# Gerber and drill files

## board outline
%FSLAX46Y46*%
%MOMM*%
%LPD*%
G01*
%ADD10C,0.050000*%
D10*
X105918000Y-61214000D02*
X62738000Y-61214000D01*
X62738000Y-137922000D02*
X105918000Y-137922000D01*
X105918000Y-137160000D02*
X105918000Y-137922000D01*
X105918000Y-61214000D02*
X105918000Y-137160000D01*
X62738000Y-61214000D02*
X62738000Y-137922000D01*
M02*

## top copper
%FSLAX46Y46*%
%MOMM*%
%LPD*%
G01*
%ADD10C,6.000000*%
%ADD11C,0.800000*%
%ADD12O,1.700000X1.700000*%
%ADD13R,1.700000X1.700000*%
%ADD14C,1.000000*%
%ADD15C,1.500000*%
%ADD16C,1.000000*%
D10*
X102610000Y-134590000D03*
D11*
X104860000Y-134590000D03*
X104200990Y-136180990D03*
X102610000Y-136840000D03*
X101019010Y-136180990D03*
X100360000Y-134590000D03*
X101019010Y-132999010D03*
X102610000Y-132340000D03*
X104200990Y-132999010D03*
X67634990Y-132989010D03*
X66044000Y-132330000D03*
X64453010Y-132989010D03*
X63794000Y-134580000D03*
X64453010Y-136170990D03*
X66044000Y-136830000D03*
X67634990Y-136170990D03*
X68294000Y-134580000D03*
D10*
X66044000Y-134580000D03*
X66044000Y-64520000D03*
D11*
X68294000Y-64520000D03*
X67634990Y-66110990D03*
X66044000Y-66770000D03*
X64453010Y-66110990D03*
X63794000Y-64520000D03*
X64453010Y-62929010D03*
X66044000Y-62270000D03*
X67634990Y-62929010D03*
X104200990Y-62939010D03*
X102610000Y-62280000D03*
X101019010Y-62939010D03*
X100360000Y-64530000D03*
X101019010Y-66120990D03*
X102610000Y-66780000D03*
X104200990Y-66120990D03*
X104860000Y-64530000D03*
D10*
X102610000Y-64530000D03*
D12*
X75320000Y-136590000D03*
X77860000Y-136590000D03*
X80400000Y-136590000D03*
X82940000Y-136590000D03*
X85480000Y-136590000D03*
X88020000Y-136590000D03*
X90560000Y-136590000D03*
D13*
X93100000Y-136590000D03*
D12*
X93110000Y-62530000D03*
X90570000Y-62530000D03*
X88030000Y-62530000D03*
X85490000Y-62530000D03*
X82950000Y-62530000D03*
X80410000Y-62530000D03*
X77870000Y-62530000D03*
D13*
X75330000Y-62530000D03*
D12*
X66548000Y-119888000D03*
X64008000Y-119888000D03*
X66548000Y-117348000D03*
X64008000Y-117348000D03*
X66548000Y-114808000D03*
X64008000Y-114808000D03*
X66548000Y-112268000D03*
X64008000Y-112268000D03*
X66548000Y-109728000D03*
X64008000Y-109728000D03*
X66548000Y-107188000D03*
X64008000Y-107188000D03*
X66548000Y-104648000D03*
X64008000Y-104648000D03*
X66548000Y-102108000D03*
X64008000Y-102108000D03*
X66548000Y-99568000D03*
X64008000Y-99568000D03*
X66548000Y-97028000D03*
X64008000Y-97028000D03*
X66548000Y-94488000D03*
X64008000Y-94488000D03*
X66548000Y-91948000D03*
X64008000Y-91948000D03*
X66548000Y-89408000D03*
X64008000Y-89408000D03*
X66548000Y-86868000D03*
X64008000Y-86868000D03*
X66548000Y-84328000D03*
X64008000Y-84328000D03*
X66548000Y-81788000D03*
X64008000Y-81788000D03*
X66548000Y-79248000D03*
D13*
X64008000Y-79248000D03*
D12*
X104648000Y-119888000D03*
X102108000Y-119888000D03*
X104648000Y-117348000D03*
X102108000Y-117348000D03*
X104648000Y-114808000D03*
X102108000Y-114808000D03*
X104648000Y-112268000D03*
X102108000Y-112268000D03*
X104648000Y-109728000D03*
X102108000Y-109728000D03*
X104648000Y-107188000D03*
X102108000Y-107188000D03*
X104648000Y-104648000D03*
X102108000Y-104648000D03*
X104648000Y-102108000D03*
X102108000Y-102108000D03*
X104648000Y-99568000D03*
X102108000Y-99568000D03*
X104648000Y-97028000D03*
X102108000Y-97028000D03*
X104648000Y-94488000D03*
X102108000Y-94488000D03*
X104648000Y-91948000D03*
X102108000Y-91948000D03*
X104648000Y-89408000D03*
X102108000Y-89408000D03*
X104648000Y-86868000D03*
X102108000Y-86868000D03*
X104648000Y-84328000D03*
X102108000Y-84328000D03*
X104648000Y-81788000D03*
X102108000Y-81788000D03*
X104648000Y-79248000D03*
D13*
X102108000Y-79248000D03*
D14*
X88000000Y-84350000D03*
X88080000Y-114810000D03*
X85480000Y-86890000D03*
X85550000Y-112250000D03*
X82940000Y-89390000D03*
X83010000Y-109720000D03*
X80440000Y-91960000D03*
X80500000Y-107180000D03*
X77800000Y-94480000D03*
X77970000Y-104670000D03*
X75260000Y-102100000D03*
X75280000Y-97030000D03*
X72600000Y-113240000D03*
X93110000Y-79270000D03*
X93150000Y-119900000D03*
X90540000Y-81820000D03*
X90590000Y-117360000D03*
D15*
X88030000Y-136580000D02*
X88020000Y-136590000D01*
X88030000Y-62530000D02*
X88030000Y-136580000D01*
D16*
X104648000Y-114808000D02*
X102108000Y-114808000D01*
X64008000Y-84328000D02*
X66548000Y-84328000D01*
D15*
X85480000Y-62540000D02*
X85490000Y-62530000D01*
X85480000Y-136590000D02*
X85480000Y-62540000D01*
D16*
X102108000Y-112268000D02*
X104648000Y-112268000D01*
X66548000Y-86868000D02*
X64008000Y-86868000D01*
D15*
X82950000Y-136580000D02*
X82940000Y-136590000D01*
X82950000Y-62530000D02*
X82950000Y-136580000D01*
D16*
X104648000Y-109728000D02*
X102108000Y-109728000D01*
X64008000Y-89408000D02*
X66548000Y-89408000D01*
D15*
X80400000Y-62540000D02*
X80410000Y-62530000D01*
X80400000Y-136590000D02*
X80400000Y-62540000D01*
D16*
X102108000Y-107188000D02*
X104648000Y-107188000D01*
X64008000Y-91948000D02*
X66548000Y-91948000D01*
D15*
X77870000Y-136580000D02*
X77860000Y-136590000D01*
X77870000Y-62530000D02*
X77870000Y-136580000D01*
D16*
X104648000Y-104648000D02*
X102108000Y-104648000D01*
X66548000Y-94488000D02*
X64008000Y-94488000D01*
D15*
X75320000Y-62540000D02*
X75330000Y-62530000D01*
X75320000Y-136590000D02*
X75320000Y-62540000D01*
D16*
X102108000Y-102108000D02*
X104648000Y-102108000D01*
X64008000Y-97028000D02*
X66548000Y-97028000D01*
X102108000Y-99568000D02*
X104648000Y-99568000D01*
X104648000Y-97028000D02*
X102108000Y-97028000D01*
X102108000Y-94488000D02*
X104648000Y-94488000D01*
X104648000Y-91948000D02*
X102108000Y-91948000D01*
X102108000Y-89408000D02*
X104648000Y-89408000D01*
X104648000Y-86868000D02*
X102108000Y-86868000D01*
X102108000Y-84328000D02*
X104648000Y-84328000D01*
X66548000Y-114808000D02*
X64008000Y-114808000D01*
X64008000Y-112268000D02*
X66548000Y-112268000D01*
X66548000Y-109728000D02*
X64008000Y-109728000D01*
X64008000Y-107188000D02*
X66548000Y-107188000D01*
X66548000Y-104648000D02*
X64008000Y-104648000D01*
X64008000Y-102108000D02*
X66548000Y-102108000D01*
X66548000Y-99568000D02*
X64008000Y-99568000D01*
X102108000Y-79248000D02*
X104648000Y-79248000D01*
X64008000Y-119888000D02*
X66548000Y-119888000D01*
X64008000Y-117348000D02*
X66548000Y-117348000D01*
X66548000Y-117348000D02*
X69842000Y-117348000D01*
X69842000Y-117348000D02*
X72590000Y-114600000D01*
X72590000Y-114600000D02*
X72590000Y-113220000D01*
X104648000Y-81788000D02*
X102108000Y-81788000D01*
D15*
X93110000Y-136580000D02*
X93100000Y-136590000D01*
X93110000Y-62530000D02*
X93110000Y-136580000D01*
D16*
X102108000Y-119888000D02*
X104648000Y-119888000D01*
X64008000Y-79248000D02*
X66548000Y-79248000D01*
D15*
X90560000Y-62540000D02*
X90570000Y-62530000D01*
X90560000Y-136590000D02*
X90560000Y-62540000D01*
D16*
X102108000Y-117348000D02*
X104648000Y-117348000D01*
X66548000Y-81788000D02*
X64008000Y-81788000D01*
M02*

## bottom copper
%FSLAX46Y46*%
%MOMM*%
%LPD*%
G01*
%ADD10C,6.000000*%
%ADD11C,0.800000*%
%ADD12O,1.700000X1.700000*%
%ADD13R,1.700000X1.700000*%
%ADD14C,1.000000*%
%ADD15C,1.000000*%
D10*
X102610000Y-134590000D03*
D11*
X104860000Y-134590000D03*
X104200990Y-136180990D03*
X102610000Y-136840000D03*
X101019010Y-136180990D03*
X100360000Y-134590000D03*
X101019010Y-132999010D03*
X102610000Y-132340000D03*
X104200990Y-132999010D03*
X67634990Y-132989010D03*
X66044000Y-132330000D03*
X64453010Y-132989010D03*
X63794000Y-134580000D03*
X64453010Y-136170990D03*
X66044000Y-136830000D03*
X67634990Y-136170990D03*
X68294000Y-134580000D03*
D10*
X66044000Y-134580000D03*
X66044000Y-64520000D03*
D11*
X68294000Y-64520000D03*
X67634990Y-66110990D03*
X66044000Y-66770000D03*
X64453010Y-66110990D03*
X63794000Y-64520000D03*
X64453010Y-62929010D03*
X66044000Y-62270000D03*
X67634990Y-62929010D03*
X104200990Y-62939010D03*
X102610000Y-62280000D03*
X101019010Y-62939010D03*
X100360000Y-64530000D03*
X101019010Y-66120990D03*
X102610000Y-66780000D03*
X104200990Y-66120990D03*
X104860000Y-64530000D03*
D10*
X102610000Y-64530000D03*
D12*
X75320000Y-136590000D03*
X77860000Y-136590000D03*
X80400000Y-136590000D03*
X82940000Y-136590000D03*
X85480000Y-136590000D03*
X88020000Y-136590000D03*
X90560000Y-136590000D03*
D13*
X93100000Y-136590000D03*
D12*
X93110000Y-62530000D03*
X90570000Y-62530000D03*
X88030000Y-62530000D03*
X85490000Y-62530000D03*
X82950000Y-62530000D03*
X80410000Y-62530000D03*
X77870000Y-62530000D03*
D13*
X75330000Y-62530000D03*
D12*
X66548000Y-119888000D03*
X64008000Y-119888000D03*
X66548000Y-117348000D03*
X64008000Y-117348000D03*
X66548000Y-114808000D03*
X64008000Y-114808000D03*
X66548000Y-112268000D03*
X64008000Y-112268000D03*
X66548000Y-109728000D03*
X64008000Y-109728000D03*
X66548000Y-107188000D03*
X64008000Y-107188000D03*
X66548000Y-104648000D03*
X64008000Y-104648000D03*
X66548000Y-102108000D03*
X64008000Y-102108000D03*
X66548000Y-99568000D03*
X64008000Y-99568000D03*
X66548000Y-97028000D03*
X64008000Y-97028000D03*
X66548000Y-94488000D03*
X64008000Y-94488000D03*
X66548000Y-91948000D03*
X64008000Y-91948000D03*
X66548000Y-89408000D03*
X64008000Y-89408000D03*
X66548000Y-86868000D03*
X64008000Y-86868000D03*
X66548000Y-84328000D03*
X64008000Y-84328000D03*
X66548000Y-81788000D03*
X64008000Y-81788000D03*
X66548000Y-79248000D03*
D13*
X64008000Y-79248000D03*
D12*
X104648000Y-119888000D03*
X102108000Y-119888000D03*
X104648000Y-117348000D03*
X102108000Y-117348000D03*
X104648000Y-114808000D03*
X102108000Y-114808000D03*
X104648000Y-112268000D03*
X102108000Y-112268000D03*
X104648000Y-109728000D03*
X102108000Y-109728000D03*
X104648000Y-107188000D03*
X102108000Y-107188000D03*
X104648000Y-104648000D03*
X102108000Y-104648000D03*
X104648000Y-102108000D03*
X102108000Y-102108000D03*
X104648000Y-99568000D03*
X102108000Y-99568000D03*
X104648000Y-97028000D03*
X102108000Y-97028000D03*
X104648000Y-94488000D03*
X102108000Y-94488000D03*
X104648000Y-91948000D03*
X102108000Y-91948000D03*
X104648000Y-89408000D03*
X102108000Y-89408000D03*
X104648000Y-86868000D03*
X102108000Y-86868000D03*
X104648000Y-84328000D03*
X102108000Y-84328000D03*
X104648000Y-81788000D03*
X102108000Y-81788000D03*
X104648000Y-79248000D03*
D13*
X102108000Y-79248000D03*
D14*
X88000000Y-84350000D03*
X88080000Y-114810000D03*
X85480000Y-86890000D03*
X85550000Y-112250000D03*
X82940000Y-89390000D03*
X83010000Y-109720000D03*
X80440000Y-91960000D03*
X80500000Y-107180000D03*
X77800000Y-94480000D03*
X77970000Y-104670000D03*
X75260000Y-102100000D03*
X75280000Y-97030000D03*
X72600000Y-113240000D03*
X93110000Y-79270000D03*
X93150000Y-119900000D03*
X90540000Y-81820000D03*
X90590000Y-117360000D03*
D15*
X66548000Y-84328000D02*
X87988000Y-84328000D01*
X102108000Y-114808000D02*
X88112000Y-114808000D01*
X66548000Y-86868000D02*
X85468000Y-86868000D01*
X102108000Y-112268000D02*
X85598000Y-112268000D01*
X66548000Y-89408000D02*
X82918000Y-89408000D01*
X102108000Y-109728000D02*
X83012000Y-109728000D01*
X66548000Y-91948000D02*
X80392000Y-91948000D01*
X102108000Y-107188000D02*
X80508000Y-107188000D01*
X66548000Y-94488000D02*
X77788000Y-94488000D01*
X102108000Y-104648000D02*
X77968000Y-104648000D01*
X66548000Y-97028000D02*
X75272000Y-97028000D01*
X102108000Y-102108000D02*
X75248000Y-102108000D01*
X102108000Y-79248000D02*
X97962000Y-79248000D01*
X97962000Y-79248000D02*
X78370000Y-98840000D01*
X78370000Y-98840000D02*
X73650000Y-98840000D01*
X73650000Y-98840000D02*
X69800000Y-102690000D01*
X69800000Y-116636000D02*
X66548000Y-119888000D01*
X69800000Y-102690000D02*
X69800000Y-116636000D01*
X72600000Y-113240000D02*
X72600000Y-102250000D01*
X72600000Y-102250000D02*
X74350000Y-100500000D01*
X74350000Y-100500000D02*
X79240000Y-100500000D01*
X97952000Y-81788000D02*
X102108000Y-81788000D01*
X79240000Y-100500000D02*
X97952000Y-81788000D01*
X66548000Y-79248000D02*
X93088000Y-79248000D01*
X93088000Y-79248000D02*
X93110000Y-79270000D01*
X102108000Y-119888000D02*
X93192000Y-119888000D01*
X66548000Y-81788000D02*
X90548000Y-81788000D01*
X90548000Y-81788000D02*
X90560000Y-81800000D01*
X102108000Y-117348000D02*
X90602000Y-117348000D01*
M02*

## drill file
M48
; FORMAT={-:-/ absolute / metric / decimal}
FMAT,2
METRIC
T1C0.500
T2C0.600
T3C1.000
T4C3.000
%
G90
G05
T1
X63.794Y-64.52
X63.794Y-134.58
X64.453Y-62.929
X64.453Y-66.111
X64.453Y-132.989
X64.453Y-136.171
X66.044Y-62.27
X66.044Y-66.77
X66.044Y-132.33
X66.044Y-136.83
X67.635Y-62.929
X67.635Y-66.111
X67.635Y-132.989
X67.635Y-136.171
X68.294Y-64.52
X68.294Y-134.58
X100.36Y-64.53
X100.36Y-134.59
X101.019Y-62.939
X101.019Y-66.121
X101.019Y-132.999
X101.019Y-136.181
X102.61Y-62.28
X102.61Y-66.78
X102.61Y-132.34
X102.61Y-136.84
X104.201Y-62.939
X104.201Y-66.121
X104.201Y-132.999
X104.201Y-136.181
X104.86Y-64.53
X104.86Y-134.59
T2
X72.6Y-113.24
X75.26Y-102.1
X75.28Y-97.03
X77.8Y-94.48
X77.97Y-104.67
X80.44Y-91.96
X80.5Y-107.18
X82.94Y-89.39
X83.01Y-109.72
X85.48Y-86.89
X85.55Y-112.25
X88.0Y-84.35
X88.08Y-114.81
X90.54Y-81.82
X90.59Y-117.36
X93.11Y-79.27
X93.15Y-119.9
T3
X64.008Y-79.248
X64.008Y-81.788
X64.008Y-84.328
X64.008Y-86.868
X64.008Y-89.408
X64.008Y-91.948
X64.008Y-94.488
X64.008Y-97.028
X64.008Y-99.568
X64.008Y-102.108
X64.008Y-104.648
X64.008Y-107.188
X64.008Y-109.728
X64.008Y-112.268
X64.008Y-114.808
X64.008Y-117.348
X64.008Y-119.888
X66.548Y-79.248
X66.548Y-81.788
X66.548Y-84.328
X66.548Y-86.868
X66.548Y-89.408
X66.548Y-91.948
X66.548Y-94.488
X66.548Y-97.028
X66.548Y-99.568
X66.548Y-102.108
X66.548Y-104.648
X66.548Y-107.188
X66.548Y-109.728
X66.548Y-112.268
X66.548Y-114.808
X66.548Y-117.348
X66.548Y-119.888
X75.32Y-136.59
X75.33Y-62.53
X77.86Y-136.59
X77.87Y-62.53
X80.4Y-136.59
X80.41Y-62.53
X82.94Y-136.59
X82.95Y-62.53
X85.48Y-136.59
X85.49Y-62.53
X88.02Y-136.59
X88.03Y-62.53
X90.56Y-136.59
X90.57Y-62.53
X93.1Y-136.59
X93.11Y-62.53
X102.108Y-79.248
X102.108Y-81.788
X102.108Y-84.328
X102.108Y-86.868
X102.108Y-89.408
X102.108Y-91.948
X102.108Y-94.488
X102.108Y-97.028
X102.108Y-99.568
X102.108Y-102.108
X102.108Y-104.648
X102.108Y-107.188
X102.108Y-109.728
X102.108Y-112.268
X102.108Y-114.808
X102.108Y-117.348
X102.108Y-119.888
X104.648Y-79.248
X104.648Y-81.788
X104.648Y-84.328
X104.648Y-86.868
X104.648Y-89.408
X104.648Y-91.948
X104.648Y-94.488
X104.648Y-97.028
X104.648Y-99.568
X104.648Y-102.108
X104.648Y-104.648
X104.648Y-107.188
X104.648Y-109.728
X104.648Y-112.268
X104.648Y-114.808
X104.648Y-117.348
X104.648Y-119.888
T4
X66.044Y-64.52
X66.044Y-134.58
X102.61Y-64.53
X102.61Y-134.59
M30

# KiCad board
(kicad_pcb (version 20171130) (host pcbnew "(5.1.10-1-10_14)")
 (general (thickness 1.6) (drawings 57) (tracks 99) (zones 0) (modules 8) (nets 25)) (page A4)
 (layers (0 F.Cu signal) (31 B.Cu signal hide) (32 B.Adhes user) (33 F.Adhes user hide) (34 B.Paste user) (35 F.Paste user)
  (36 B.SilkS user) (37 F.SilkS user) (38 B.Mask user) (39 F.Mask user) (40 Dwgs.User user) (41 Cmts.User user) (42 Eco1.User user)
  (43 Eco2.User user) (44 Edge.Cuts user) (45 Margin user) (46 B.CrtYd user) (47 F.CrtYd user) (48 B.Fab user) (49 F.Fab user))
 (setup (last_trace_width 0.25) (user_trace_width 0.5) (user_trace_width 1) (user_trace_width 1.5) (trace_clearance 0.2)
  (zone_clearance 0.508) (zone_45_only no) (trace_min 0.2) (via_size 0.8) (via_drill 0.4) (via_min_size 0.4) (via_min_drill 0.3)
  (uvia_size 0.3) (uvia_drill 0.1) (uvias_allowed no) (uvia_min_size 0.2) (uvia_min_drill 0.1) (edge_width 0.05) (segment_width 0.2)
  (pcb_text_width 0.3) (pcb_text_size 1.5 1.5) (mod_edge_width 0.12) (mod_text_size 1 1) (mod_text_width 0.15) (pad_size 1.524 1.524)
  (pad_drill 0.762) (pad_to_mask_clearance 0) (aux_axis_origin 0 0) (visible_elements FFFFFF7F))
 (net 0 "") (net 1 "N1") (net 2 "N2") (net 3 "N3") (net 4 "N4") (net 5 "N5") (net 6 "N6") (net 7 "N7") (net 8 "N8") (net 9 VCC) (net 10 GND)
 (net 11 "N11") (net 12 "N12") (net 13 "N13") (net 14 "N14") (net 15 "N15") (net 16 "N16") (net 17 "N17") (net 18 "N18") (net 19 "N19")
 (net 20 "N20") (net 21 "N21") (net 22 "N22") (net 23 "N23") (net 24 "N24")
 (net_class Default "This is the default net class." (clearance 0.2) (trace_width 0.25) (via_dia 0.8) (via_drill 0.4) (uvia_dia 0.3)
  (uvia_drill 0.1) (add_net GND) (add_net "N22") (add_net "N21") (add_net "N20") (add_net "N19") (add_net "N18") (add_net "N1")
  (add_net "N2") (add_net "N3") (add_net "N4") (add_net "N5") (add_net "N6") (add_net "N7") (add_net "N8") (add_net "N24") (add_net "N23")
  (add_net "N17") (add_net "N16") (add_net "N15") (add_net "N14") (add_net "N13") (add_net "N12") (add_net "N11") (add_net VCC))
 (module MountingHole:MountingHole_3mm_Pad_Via (layer F.Cu) (at 102.61 134.59)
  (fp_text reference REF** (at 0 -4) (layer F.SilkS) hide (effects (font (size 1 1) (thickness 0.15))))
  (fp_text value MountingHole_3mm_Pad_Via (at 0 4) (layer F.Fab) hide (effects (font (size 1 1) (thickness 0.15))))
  (pad 1 thru_hole circle (at 0 0) (size 6 6) (drill 3) (layers *.Cu *.Mask))
  (pad 1 thru_hole circle (at 2.25 0) (size 0.8 0.8) (drill 0.5) (layers *.Cu *.Mask))
  (pad 1 thru_hole circle (at 1.59099 1.59099) (size 0.8 0.8) (drill 0.5) (layers *.Cu *.Mask))
  (pad 1 thru_hole circle (at 0 2.25) (size 0.8 0.8) (drill 0.5) (layers *.Cu *.Mask))
  (pad 1 thru_hole circle (at -1.59099 1.59099) (size 0.8 0.8) (drill 0.5) (layers *.Cu *.Mask))
  (pad 1 thru_hole circle (at -2.25 0) (size 0.8 0.8) (drill 0.5) (layers *.Cu *.Mask))
  (pad 1 thru_hole circle (at -1.59099 -1.59099) (size 0.8 0.8) (drill 0.5) (layers *.Cu *.Mask))
  (pad 1 thru_hole circle (at 0 -2.25) (size 0.8 0.8) (drill 0.5) (layers *.Cu *.Mask))
  (pad 1 thru_hole circle (at 1.59099 -1.59099) (size 0.8 0.8) (drill 0.5) (layers *.Cu *.Mask)))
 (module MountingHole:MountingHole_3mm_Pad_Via (layer F.Cu) (at 66.044 134.58)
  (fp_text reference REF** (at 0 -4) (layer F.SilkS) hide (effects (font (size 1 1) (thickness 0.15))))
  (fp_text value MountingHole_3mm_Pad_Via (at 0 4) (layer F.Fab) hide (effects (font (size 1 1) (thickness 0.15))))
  (pad 1 thru_hole circle (at 1.59099 -1.59099) (size 0.8 0.8) (drill 0.5) (layers *.Cu *.Mask))
  (pad 1 thru_hole circle (at 0 -2.25) (size 0.8 0.8) (drill 0.5) (layers *.Cu *.Mask))
  (pad 1 thru_hole circle (at -1.59099 -1.59099) (size 0.8 0.8) (drill 0.5) (layers *.Cu *.Mask))
  (pad 1 thru_hole circle (at -2.25 0) (size 0.8 0.8) (drill 0.5) (layers *.Cu *.Mask))
  (pad 1 thru_hole circle (at -1.59099 1.59099) (size 0.8 0.8) (drill 0.5) (layers *.Cu *.Mask))
  (pad 1 thru_hole circle (at 0 2.25) (size 0.8 0.8) (drill 0.5) (layers *.Cu *.Mask))
  (pad 1 thru_hole circle (at 1.59099 1.59099) (size 0.8 0.8) (drill 0.5) (layers *.Cu *.Mask))
  (pad 1 thru_hole circle (at 2.25 0) (size 0.8 0.8) (drill 0.5) (layers *.Cu *.Mask))
  (pad 1 thru_hole circle (at 0 0) (size 6 6) (drill 3) (layers *.Cu *.Mask)))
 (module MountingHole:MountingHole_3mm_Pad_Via (layer F.Cu) (at 66.044 64.52)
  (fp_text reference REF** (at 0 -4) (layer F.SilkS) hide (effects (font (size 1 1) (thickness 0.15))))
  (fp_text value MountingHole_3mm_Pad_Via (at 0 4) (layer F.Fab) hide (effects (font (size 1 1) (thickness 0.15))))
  (pad 1 thru_hole circle (at 0 0) (size 6 6) (drill 3) (layers *.Cu *.Mask))
  (pad 1 thru_hole circle (at 2.25 0) (size 0.8 0.8) (drill 0.5) (layers *.Cu *.Mask))
  (pad 1 thru_hole circle (at 1.59099 1.59099) (size 0.8 0.8) (drill 0.5) (layers *.Cu *.Mask))
  (pad 1 thru_hole circle (at 0 2.25) (size 0.8 0.8) (drill 0.5) (layers *.Cu *.Mask))
  (pad 1 thru_hole circle (at -1.59099 1.59099) (size 0.8 0.8) (drill 0.5) (layers *.Cu *.Mask))
  (pad 1 thru_hole circle (at -2.25 0) (size 0.8 0.8) (drill 0.5) (layers *.Cu *.Mask))
  (pad 1 thru_hole circle (at -1.59099 -1.59099) (size 0.8 0.8) (drill 0.5) (layers *.Cu *.Mask))
  (pad 1 thru_hole circle (at 0 -2.25) (size 0.8 0.8) (drill 0.5) (layers *.Cu *.Mask))
  (pad 1 thru_hole circle (at 1.59099 -1.59099) (size 0.8 0.8) (drill 0.5) (layers *.Cu *.Mask)))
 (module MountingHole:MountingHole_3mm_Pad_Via (layer F.Cu) (at 102.61 64.53)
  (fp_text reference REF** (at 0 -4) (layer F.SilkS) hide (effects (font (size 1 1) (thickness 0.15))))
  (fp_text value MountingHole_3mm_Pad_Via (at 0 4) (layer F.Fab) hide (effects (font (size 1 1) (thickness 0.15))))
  (pad 1 thru_hole circle (at 1.59099 -1.59099) (size 0.8 0.8) (drill 0.5) (layers *.Cu *.Mask))
  (pad 1 thru_hole circle (at 0 -2.25) (size 0.8 0.8) (drill 0.5) (layers *.Cu *.Mask))
  (pad 1 thru_hole circle (at -1.59099 -1.59099) (size 0.8 0.8) (drill 0.5) (layers *.Cu *.Mask))
  (pad 1 thru_hole circle (at -2.25 0) (size 0.8 0.8) (drill 0.5) (layers *.Cu *.Mask))
  (pad 1 thru_hole circle (at -1.59099 1.59099) (size 0.8 0.8) (drill 0.5) (layers *.Cu *.Mask))
  (pad 1 thru_hole circle (at 0 2.25) (size 0.8 0.8) (drill 0.5) (layers *.Cu *.Mask))
  (pad 1 thru_hole circle (at 1.59099 1.59099) (size 0.8 0.8) (drill 0.5) (layers *.Cu *.Mask))
  (pad 1 thru_hole circle (at 2.25 0) (size 0.8 0.8) (drill 0.5) (layers *.Cu *.Mask))
  (pad 1 thru_hole circle (at 0 0) (size 6 6) (drill 3) (layers *.Cu *.Mask)))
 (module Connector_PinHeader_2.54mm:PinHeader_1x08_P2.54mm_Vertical (layer F.Cu) (at 93.1 136.59 270)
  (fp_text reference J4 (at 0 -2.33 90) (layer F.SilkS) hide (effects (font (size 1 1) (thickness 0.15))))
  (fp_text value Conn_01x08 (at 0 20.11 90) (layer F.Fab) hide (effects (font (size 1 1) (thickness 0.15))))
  (pad 8 thru_hole oval (at 0 17.78 270) (size 1.7 1.7) (drill 1) (layers *.Cu *.Mask) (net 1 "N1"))
  (pad 7 thru_hole oval (at 0 15.24 270) (size 1.7 1.7) (drill 1) (layers *.Cu *.Mask) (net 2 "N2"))
  (pad 6 thru_hole oval (at 0 12.7 270) (size 1.7 1.7) (drill 1) (layers *.Cu *.Mask) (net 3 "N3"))
  (pad 5 thru_hole oval (at 0 10.16 270) (size 1.7 1.7) (drill 1) (layers *.Cu *.Mask) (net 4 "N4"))
  (pad 4 thru_hole oval (at 0 7.62 270) (size 1.7 1.7) (drill 1) (layers *.Cu *.Mask) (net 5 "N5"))
  (pad 3 thru_hole oval (at 0 5.08 270) (size 1.7 1.7) (drill 1) (layers *.Cu *.Mask) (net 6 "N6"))
  (pad 2 thru_hole oval (at 0 2.54 270) (size 1.7 1.7) (drill 1) (layers *.Cu *.Mask) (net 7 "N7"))
  (pad 1 thru_hole rect (at 0 0 270) (size 1.7 1.7) (drill 1) (layers *.Cu *.Mask) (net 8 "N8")))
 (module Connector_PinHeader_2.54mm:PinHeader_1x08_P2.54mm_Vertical (layer F.Cu) (at 75.33 62.53 90)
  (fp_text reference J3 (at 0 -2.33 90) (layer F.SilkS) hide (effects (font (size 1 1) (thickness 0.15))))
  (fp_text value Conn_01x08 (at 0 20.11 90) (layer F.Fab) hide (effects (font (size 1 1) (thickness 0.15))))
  (pad 8 thru_hole oval (at 0 17.78 90) (size 1.7 1.7) (drill 1) (layers *.Cu *.Mask) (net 8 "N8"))
  (pad 7 thru_hole oval (at 0 15.24 90) (size 1.7 1.7) (drill 1) (layers *.Cu *.Mask) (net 7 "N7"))
  (pad 6 thru_hole oval (at 0 12.7 90) (size 1.7 1.7) (drill 1) (layers *.Cu *.Mask) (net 6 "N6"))
  (pad 5 thru_hole oval (at 0 10.16 90) (size 1.7 1.7) (drill 1) (layers *.Cu *.Mask) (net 5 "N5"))
  (pad 4 thru_hole oval (at 0 7.62 90) (size 1.7 1.7) (drill 1) (layers *.Cu *.Mask) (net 4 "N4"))
  (pad 3 thru_hole oval (at 0 5.08 90) (size 1.7 1.7) (drill 1) (layers *.Cu *.Mask) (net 3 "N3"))
  (pad 2 thru_hole oval (at 0 2.54 90) (size 1.7 1.7) (drill 1) (layers *.Cu *.Mask) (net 2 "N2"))
  (pad 1 thru_hole rect (at 0 0 90) (size 1.7 1.7) (drill 1) (layers *.Cu *.Mask) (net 1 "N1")))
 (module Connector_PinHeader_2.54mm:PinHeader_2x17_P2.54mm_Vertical (layer F.Cu) (at 64.008 79.248)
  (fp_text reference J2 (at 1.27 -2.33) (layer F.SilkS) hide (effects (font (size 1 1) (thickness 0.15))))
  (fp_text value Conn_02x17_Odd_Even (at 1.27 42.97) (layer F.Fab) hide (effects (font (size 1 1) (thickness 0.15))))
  (pad 34 thru_hole oval (at 2.54 40.64) (size 1.7 1.7) (drill 1) (layers *.Cu *.Mask) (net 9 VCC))
  (pad 33 thru_hole oval (at 0 40.64) (size 1.7 1.7) (drill 1) (layers *.Cu *.Mask) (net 9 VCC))
  (pad 32 thru_hole oval (at 2.54 38.1) (size 1.7 1.7) (drill 1) (layers *.Cu *.Mask) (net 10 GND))
  (pad 31 thru_hole oval (at 0 38.1) (size 1.7 1.7) (drill 1) (layers *.Cu *.Mask) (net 10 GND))
  (pad 30 thru_hole oval (at 2.54 35.56) (size 1.7 1.7) (drill 1) (layers *.Cu *.Mask) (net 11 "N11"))
  (pad 29 thru_hole oval (at 0 35.56) (size 1.7 1.7) (drill 1) (layers *.Cu *.Mask) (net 11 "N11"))
  (pad 28 thru_hole oval (at 2.54 33.02) (size 1.7 1.7) (drill 1) (layers *.Cu *.Mask) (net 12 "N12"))
  (pad 27 thru_hole oval (at 0 33.02) (size 1.7 1.7) (drill 1) (layers *.Cu *.Mask) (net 12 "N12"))
  (pad 26 thru_hole oval (at 2.54 30.48) (size 1.7 1.7) (drill 1) (layers *.Cu *.Mask) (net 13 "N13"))
  (pad 25 thru_hole oval (at 0 30.48) (size 1.7 1.7) (drill 1) (layers *.Cu *.Mask) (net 13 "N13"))
  (pad 24 thru_hole oval (at 2.54 27.94) (size 1.7 1.7) (drill 1) (layers *.Cu *.Mask) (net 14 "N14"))
  (pad 23 thru_hole oval (at 0 27.94) (size 1.7 1.7) (drill 1) (layers *.Cu *.Mask) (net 14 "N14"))
  (pad 22 thru_hole oval (at 2.54 25.4) (size 1.7 1.7) (drill 1) (layers *.Cu *.Mask) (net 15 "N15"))
  (pad 21 thru_hole oval (at 0 25.4) (size 1.7 1.7) (drill 1) (layers *.Cu *.Mask) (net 15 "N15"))
  (pad 20 thru_hole oval (at 2.54 22.86) (size 1.7 1.7) (drill 1) (layers *.Cu *.Mask) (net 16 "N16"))
  (pad 19 thru_hole oval (at 0 22.86) (size 1.7 1.7) (drill 1) (layers *.Cu *.Mask) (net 16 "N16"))
  (pad 18 thru_hole oval (at 2.54 20.32) (size 1.7 1.7) (drill 1) (layers *.Cu *.Mask) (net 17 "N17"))
  (pad 17 thru_hole oval (at 0 20.32) (size 1.7 1.7) (drill 1) (layers *.Cu *.Mask) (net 17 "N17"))
  (pad 16 thru_hole oval (at 2.54 17.78) (size 1.7 1.7) (drill 1) (layers *.Cu *.Mask) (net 1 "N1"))
  (pad 15 thru_hole oval (at 0 17.78) (size 1.7 1.7) (drill 1) (layers *.Cu *.Mask) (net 1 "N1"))
  (pad 14 thru_hole oval (at 2.54 15.24) (size 1.7 1.7) (drill 1) (layers *.Cu *.Mask) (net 2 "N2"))
  (pad 13 thru_hole oval (at 0 15.24) (size 1.7 1.7) (drill 1) (layers *.Cu *.Mask) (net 2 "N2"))
  (pad 12 thru_hole oval (at 2.54 12.7) (size 1.7 1.7) (drill 1) (layers *.Cu *.Mask) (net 3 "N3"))
  (pad 11 thru_hole oval (at 0 12.7) (size 1.7 1.7) (drill 1) (layers *.Cu *.Mask) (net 3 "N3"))
  (pad 10 thru_hole oval (at 2.54 10.16) (size 1.7 1.7) (drill 1) (layers *.Cu *.Mask) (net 4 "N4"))
  (pad 9 thru_hole oval (at 0 10.16) (size 1.7 1.7) (drill 1) (layers *.Cu *.Mask) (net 4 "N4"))
  (pad 8 thru_hole oval (at 2.54 7.62) (size 1.7 1.7) (drill 1) (layers *.Cu *.Mask) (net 5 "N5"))
  (pad 7 thru_hole oval (at 0 7.62) (size 1.7 1.7) (drill 1) (layers *.Cu *.Mask) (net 5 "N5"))
  (pad 6 thru_hole oval (at 2.54 5.08) (size 1.7 1.7) (drill 1) (layers *.Cu *.Mask) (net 6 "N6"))
  (pad 5 thru_hole oval (at 0 5.08) (size 1.7 1.7) (drill 1) (layers *.Cu *.Mask) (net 6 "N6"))
  (pad 4 thru_hole oval (at 2.54 2.54) (size 1.7 1.7) (drill 1) (layers *.Cu *.Mask) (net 7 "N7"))
  (pad 3 thru_hole oval (at 0 2.54) (size 1.7 1.7) (drill 1) (layers *.Cu *.Mask) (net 7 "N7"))
  (pad 2 thru_hole oval (at 2.54 0) (size 1.7 1.7) (drill 1) (layers *.Cu *.Mask) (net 8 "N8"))
  (pad 1 thru_hole rect (at 0 0) (size 1.7 1.7) (drill 1) (layers *.Cu *.Mask) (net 8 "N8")))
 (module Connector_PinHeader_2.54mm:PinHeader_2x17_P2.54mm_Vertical (layer F.Cu) (at 102.108 79.248)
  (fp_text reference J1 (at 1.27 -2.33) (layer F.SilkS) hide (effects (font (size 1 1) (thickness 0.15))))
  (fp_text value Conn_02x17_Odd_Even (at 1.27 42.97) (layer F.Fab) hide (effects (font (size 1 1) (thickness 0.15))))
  (pad 34 thru_hole oval (at 2.54 40.64) (size 1.7 1.7) (drill 1) (layers *.Cu *.Mask) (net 8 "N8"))
  (pad 33 thru_hole oval (at 0 40.64) (size 1.7 1.7) (drill 1) (layers *.Cu *.Mask) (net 8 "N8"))
  (pad 32 thru_hole oval (at 2.54 38.1) (size 1.7 1.7) (drill 1) (layers *.Cu *.Mask) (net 7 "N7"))
  (pad 31 thru_hole oval (at 0 38.1) (size 1.7 1.7) (drill 1) (layers *.Cu *.Mask) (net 7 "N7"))
  (pad 30 thru_hole oval (at 2.54 35.56) (size 1.7 1.7) (drill 1) (layers *.Cu *.Mask) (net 6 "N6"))
  (pad 29 thru_hole oval (at 0 35.56) (size 1.7 1.7) (drill 1) (layers *.Cu *.Mask) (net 6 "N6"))
  (pad 28 thru_hole oval (at 2.54 33.02) (size 1.7 1.7) (drill 1) (layers *.Cu *.Mask) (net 5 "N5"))
  (pad 27 thru_hole oval (at 0 33.02) (size 1.7 1.7) (drill 1) (layers *.Cu *.Mask) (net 5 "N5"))
  (pad 26 thru_hole oval (at 2.54 30.48) (size 1.7 1.7) (drill 1) (layers *.Cu *.Mask) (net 4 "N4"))
  (pad 25 thru_hole oval (at 0 30.48) (size 1.7 1.7) (drill 1) (layers *.Cu *.Mask) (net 4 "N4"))
  (pad 24 thru_hole oval (at 2.54 27.94) (size 1.7 1.7) (drill 1) (layers *.Cu *.Mask) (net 3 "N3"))
  (pad 23 thru_hole oval (at 0 27.94) (size 1.7 1.7) (drill 1) (layers *.Cu *.Mask) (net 3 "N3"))
  (pad 22 thru_hole oval (at 2.54 25.4) (size 1.7 1.7) (drill 1) (layers *.Cu *.Mask) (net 2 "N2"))
  (pad 21 thru_hole oval (at 0 25.4) (size 1.7 1.7) (drill 1) (layers *.Cu *.Mask) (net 2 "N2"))
  (pad 20 thru_hole oval (at 2.54 22.86) (size 1.7 1.7) (drill 1) (layers *.Cu *.Mask) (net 1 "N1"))
  (pad 19 thru_hole oval (at 0 22.86) (size 1.7 1.7) (drill 1) (layers *.Cu *.Mask) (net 1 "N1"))
  (pad 18 thru_hole oval (at 2.54 20.32) (size 1.7 1.7) (drill 1) (layers *.Cu *.Mask) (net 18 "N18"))
  (pad 17 thru_hole oval (at 0 20.32) (size 1.7 1.7) (drill 1) (layers *.Cu *.Mask) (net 18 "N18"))
  (pad 16 thru_hole oval (at 2.54 17.78) (size 1.7 1.7) (drill 1) (layers *.Cu *.Mask) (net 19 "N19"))
  (pad 15 thru_hole oval (at 0 17.78) (size 1.7 1.7) (drill 1) (layers *.Cu *.Mask) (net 19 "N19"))
  (pad 14 thru_hole oval (at 2.54 15.24) (size 1.7 1.7) (drill 1) (layers *.Cu *.Mask) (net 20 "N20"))
  (pad 13 thru_hole oval (at 0 15.24) (size 1.7 1.7) (drill 1) (layers *.Cu *.Mask) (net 20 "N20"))
  (pad 12 thru_hole oval (at 2.54 12.7) (size 1.7 1.7) (drill 1) (layers *.Cu *.Mask) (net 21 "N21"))
  (pad 11 thru_hole oval (at 0 12.7) (size 1.7 1.7) (drill 1) (layers *.Cu *.Mask) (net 21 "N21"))
  (pad 10 thru_hole oval (at 2.54 10.16) (size 1.7 1.7) (drill 1) (layers *.Cu *.Mask) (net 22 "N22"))
  (pad 9 thru_hole oval (at 0 10.16) (size 1.7 1.7) (drill 1) (layers *.Cu *.Mask) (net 22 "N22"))
  (pad 8 thru_hole oval (at 2.54 7.62) (size 1.7 1.7) (drill 1) (layers *.Cu *.Mask) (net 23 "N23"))
  (pad 7 thru_hole oval (at 0 7.62) (size 1.7 1.7) (drill 1) (layers *.Cu *.Mask) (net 23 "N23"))
  (pad 6 thru_hole oval (at 2.54 5.08) (size 1.7 1.7) (drill 1) (layers *.Cu *.Mask) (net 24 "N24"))
  (pad 5 thru_hole oval (at 0 5.08) (size 1.7 1.7) (drill 1) (layers *.Cu *.Mask) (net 24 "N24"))
  (pad 4 thru_hole oval (at 2.54 2.54) (size 1.7 1.7) (drill 1) (layers *.Cu *.Mask) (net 10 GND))
  (pad 3 thru_hole oval (at 0 2.54) (size 1.7 1.7) (drill 1) (layers *.Cu *.Mask) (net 10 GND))
  (pad 2 thru_hole oval (at 2.54 0) (size 1.7 1.7) (drill 1) (layers *.Cu *.Mask) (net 9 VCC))
  (pad 1 thru_hole rect (at 0 0) (size 1.7 1.7) (drill 1) (layers *.Cu *.Mask) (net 9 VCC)))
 (gr_line (start 105.918 61.214) (end 62.738 61.214) (layer Edge.Cuts) (width 0.05))
 (gr_line (start 62.738 137.922) (end 105.918 137.922) (layer Edge.Cuts) (width 0.05))
 (gr_line (start 105.918 137.16) (end 105.918 137.922) (layer Edge.Cuts) (width 0.05))
 (gr_line (start 105.918 61.214) (end 105.918 137.16) (layer Edge.Cuts) (width 0.05))
 (gr_line (start 62.738 61.214) (end 62.738 137.922) (layer Edge.Cuts) (width 0.05))
 (segment (start 88.03 136.58) (end 88.02 136.59) (width 1.5) (layer F.Cu) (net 6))
 (segment (start 88.03 62.53) (end 88.03 136.58) (width 1.5) (layer F.Cu) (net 6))
 (segment (start 66.548 84.328) (end 87.988 84.328) (width 1) (layer B.Cu) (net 6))
 (via (at 88 84.35) (size 1) (drill 0.6) (layers F.Cu B.Cu) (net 6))
 (segment (start 102.108 114.808) (end 88.112 114.808) (width 1) (layer B.Cu) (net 6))
 (via (at 88.08 114.81) (size 1) (drill 0.6) (layers F.Cu B.Cu) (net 6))
 (segment (start 104.648 114.808) (end 102.108 114.808) (width 1) (layer F.Cu) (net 6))
 (segment (start 64.008 84.328) (end 66.548 84.328) (width 1) (layer F.Cu) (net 6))
 (segment (start 85.48 62.54) (end 85.49 62.53) (width 1.5) (layer F.Cu) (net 5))
 (segment (start 85.48 136.59) (end 85.48 62.54) (width 1.5) (layer F.Cu) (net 5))
 (via (at 85.48 86.89) (size 1) (drill 0.6) (layers F.Cu B.Cu) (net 5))
 (segment (start 66.548 86.868) (end 85.468 86.868) (width 1) (layer B.Cu) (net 5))
 (segment (start 102.108 112.268) (end 85.598 112.268) (width 1) (layer B.Cu) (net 5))
 (via (at 85.55 112.25) (size 1) (drill 0.6) (layers F.Cu B.Cu) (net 5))
 (segment (start 102.108 112.268) (end 104.648 112.268) (width 1) (layer F.Cu) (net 5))
 (segment (start 66.548 86.868) (end 64.008 86.868) (width 1) (layer F.Cu) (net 5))
 (segment (start 82.95 136.58) (end 82.94 136.59) (width 1.5) (layer F.Cu) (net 4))
 (segment (start 82.95 62.53) (end 82.95 136.58) (width 1.5) (layer F.Cu) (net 4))
 (via (at 82.94 89.39) (size 1) (drill 0.6) (layers F.Cu B.Cu) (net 4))
 (segment (start 66.548 89.408) (end 82.918 89.408) (width 1) (layer B.Cu) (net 4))
 (segment (start 102.108 109.728) (end 83.012 109.728) (width 1) (layer B.Cu) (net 4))
 (via (at 83.01 109.72) (size 1) (drill 0.6) (layers F.Cu B.Cu) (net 4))
 (segment (start 104.648 109.728) (end 102.108 109.728) (width 1) (layer F.Cu) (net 4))
 (segment (start 64.008 89.408) (end 66.548 89.408) (width 1) (layer F.Cu) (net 4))
 (segment (start 80.4 62.54) (end 80.41 62.53) (width 1.5) (layer F.Cu) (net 3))
 (segment (start 80.4 136.59) (end 80.4 62.54) (width 1.5) (layer F.Cu) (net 3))
 (via (at 80.44 91.96) (size 1) (drill 0.6) (layers F.Cu B.Cu) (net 3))
 (segment (start 66.548 91.948) (end 80.392 91.948) (width 1) (layer B.Cu) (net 3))
 (segment (start 102.108 107.188) (end 80.508 107.188) (width 1) (layer B.Cu) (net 3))
 (via (at 80.5 107.18) (size 1) (drill 0.6) (layers F.Cu B.Cu) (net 3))
 (segment (start 102.108 107.188) (end 104.648 107.188) (width 1) (layer F.Cu) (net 3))
 (segment (start 64.008 91.948) (end 66.548 91.948) (width 1) (layer F.Cu) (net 3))
 (segment (start 77.87 136.58) (end 77.86 136.59) (width 1.5) (layer F.Cu) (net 2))
 (segment (start 77.87 62.53) (end 77.87 136.58) (width 1.5) (layer F.Cu) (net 2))
 (via (at 77.8 94.48) (size 1) (drill 0.6) (layers F.Cu B.Cu) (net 2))
 (segment (start 66.548 94.488) (end 77.788 94.488) (width 1) (layer B.Cu) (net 2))
 (segment (start 102.108 104.648) (end 77.968 104.648) (width 1) (layer B.Cu) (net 2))
 (via (at 77.97 104.67) (size 1) (drill 0.6) (layers F.Cu B.Cu) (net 2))
 (segment (start 104.648 104.648) (end 102.108 104.648) (width 1) (layer F.Cu) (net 2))
 (segment (start 66.548 94.488) (end 64.008 94.488) (width 1) (layer F.Cu) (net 2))
 (segment (start 75.32 62.54) (end 75.33 62.53) (width 1.5) (layer F.Cu) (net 1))
 (segment (start 75.32 136.59) (end 75.32 62.54) (width 1.5) (layer F.Cu) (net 1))
 (via (at 75.26 102.1) (size 1) (drill 0.6) (layers F.Cu B.Cu) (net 1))
 (via (at 75.28 97.03) (size 1) (drill 0.6) (layers F.Cu B.Cu) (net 1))
 (segment (start 66.548 97.028) (end 75.272 97.028) (width 1) (layer B.Cu) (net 1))
 (segment (start 102.108 102.108) (end 75.248 102.108) (width 1) (layer B.Cu) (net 1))
 (segment (start 102.108 102.108) (end 104.648 102.108) (width 1) (layer F.Cu) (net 1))
 (segment (start 64.008 97.028) (end 66.548 97.028) (width 1) (layer F.Cu) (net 1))
 (segment (start 102.108 99.568) (end 104.648 99.568) (width 1) (layer F.Cu) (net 18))
 (segment (start 104.648 97.028) (end 102.108 97.028) (width 1) (layer F.Cu) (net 19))
 (segment (start 102.108 94.488) (end 104.648 94.488) (width 1) (layer F.Cu) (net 20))
 (segment (start 104.648 91.948) (end 102.108 91.948) (width 1) (layer F.Cu) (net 21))
 (segment (start 102.108 89.408) (end 104.648 89.408) (width 1) (layer F.Cu) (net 22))
 (segment (start 104.648 86.868) (end 102.108 86.868) (width 1) (layer F.Cu) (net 23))
 (segment (start 102.108 84.328) (end 104.648 84.328) (width 1) (layer F.Cu) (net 24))
 (segment (start 66.548 114.808) (end 64.008 114.808) (width 1) (layer F.Cu) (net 11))
 (segment (start 64.008 112.268) (end 66.548 112.268) (width 1) (layer F.Cu) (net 12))
 (segment (start 66.548 109.728) (end 64.008 109.728) (width 1) (layer F.Cu) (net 13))
 (segment (start 64.008 107.188) (end 66.548 107.188) (width 1) (layer F.Cu) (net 14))
 (segment (start 66.548 104.648) (end 64.008 104.648) (width 1) (layer F.Cu) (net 15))
 (segment (start 64.008 102.108) (end 66.548 102.108) (width 1) (layer F.Cu) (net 16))
 (segment (start 66.548 99.568) (end 64.008 99.568) (width 1) (layer F.Cu) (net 17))
 (segment (start 102.108 79.248) (end 97.962 79.248) (width 1) (layer B.Cu) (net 9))
 (segment (start 97.962 79.248) (end 78.37 98.84) (width 1) (layer B.Cu) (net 9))
 (segment (start 78.37 98.84) (end 73.65 98.84) (width 1) (layer B.Cu) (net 9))
 (segment (start 73.65 98.84) (end 69.8 102.69) (width 1) (layer B.Cu) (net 9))
 (segment (start 69.8 116.636) (end 66.548 119.888) (width 1) (layer B.Cu) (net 9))
 (segment (start 69.8 102.69) (end 69.8 116.636) (width 1) (layer B.Cu) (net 9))
 (segment (start 102.108 79.248) (end 104.648 79.248) (width 1) (layer F.Cu) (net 9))
 (segment (start 64.008 119.888) (end 66.548 119.888) (width 1) (layer F.Cu) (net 9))
 (via (at 72.6 113.24) (size 1) (drill 0.6) (layers F.Cu B.Cu) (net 10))
 (segment (start 64.008 117.348) (end 66.548 117.348) (width 1) (layer F.Cu) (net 10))
 (segment (start 66.548 117.348) (end 69.842 117.348) (width 1) (layer F.Cu) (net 10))
 (segment (start 69.842 117.348) (end 72.59 114.6) (width 1) (layer F.Cu) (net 10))
 (segment (start 72.59 114.6) (end 72.59 113.22) (width 1) (layer F.Cu) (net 10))
 (segment (start 72.6 113.24) (end 72.6 102.25) (width 1) (layer B.Cu) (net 10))
 (segment (start 72.6 102.25) (end 74.35 100.5) (width 1) (layer B.Cu) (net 10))
 (segment (start 74.35 100.5) (end 79.24 100.5) (width 1) (layer B.Cu) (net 10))
 (segment (start 97.952 81.788) (end 102.108 81.788) (width 1) (layer B.Cu) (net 10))
 (segment (start 79.24 100.5) (end 97.952 81.788) (width 1) (layer B.Cu) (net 10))
 (segment (start 104.648 81.788) (end 102.108 81.788) (width 1) (layer F.Cu) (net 10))
 (segment (start 93.11 136.58) (end 93.1 136.59) (width 1.5) (layer F.Cu) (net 8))
 (segment (start 93.11 62.53) (end 93.11 136.58) (width 1.5) (layer F.Cu) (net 8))
 (via (at 93.11 79.27) (size 1) (drill 0.6) (layers F.Cu B.Cu) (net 8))
 (segment (start 66.548 79.248) (end 93.088 79.248) (width 1) (layer B.Cu) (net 8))
 (segment (start 93.088 79.248) (end 93.11 79.27) (width 1) (layer B.Cu) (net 8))
 (segment (start 102.108 119.888) (end 93.192 119.888) (width 1) (layer B.Cu) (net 8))
 (via (at 93.15 119.9) (size 1) (drill 0.6) (layers F.Cu B.Cu) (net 8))
 (segment (start 102.108 119.888) (end 104.648 119.888) (width 1) (layer F.Cu) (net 8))
 (segment (start 64.008 79.248) (end 66.548 79.248) (width 1) (layer F.Cu) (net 8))
 (via (at 90.54 81.82) (size 1) (drill 0.6) (layers F.Cu B.Cu) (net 7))
 (segment (start 90.56 62.54) (end 90.57 62.53) (width 1.5) (layer F.Cu) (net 7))
 (segment (start 90.56 136.59) (end 90.56 62.54) (width 1.5) (layer F.Cu) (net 7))
 (segment (start 66.548 81.788) (end 90.548 81.788) (width 1) (layer B.Cu) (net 7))
 (segment (start 90.548 81.788) (end 90.56 81.8) (width 1) (layer B.Cu) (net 7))
 (via (at 90.59 117.36) (size 1) (drill 0.6) (layers F.Cu B.Cu) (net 7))
 (segment (start 102.108 117.348) (end 90.602 117.348) (width 1) (layer B.Cu) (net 7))
 (segment (start 102.108 117.348) (end 104.648 117.348) (width 1) (layer F.Cu) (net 7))
 (segment (start 66.548 81.788) (end 64.008 81.788) (width 1) (layer F.Cu) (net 7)))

